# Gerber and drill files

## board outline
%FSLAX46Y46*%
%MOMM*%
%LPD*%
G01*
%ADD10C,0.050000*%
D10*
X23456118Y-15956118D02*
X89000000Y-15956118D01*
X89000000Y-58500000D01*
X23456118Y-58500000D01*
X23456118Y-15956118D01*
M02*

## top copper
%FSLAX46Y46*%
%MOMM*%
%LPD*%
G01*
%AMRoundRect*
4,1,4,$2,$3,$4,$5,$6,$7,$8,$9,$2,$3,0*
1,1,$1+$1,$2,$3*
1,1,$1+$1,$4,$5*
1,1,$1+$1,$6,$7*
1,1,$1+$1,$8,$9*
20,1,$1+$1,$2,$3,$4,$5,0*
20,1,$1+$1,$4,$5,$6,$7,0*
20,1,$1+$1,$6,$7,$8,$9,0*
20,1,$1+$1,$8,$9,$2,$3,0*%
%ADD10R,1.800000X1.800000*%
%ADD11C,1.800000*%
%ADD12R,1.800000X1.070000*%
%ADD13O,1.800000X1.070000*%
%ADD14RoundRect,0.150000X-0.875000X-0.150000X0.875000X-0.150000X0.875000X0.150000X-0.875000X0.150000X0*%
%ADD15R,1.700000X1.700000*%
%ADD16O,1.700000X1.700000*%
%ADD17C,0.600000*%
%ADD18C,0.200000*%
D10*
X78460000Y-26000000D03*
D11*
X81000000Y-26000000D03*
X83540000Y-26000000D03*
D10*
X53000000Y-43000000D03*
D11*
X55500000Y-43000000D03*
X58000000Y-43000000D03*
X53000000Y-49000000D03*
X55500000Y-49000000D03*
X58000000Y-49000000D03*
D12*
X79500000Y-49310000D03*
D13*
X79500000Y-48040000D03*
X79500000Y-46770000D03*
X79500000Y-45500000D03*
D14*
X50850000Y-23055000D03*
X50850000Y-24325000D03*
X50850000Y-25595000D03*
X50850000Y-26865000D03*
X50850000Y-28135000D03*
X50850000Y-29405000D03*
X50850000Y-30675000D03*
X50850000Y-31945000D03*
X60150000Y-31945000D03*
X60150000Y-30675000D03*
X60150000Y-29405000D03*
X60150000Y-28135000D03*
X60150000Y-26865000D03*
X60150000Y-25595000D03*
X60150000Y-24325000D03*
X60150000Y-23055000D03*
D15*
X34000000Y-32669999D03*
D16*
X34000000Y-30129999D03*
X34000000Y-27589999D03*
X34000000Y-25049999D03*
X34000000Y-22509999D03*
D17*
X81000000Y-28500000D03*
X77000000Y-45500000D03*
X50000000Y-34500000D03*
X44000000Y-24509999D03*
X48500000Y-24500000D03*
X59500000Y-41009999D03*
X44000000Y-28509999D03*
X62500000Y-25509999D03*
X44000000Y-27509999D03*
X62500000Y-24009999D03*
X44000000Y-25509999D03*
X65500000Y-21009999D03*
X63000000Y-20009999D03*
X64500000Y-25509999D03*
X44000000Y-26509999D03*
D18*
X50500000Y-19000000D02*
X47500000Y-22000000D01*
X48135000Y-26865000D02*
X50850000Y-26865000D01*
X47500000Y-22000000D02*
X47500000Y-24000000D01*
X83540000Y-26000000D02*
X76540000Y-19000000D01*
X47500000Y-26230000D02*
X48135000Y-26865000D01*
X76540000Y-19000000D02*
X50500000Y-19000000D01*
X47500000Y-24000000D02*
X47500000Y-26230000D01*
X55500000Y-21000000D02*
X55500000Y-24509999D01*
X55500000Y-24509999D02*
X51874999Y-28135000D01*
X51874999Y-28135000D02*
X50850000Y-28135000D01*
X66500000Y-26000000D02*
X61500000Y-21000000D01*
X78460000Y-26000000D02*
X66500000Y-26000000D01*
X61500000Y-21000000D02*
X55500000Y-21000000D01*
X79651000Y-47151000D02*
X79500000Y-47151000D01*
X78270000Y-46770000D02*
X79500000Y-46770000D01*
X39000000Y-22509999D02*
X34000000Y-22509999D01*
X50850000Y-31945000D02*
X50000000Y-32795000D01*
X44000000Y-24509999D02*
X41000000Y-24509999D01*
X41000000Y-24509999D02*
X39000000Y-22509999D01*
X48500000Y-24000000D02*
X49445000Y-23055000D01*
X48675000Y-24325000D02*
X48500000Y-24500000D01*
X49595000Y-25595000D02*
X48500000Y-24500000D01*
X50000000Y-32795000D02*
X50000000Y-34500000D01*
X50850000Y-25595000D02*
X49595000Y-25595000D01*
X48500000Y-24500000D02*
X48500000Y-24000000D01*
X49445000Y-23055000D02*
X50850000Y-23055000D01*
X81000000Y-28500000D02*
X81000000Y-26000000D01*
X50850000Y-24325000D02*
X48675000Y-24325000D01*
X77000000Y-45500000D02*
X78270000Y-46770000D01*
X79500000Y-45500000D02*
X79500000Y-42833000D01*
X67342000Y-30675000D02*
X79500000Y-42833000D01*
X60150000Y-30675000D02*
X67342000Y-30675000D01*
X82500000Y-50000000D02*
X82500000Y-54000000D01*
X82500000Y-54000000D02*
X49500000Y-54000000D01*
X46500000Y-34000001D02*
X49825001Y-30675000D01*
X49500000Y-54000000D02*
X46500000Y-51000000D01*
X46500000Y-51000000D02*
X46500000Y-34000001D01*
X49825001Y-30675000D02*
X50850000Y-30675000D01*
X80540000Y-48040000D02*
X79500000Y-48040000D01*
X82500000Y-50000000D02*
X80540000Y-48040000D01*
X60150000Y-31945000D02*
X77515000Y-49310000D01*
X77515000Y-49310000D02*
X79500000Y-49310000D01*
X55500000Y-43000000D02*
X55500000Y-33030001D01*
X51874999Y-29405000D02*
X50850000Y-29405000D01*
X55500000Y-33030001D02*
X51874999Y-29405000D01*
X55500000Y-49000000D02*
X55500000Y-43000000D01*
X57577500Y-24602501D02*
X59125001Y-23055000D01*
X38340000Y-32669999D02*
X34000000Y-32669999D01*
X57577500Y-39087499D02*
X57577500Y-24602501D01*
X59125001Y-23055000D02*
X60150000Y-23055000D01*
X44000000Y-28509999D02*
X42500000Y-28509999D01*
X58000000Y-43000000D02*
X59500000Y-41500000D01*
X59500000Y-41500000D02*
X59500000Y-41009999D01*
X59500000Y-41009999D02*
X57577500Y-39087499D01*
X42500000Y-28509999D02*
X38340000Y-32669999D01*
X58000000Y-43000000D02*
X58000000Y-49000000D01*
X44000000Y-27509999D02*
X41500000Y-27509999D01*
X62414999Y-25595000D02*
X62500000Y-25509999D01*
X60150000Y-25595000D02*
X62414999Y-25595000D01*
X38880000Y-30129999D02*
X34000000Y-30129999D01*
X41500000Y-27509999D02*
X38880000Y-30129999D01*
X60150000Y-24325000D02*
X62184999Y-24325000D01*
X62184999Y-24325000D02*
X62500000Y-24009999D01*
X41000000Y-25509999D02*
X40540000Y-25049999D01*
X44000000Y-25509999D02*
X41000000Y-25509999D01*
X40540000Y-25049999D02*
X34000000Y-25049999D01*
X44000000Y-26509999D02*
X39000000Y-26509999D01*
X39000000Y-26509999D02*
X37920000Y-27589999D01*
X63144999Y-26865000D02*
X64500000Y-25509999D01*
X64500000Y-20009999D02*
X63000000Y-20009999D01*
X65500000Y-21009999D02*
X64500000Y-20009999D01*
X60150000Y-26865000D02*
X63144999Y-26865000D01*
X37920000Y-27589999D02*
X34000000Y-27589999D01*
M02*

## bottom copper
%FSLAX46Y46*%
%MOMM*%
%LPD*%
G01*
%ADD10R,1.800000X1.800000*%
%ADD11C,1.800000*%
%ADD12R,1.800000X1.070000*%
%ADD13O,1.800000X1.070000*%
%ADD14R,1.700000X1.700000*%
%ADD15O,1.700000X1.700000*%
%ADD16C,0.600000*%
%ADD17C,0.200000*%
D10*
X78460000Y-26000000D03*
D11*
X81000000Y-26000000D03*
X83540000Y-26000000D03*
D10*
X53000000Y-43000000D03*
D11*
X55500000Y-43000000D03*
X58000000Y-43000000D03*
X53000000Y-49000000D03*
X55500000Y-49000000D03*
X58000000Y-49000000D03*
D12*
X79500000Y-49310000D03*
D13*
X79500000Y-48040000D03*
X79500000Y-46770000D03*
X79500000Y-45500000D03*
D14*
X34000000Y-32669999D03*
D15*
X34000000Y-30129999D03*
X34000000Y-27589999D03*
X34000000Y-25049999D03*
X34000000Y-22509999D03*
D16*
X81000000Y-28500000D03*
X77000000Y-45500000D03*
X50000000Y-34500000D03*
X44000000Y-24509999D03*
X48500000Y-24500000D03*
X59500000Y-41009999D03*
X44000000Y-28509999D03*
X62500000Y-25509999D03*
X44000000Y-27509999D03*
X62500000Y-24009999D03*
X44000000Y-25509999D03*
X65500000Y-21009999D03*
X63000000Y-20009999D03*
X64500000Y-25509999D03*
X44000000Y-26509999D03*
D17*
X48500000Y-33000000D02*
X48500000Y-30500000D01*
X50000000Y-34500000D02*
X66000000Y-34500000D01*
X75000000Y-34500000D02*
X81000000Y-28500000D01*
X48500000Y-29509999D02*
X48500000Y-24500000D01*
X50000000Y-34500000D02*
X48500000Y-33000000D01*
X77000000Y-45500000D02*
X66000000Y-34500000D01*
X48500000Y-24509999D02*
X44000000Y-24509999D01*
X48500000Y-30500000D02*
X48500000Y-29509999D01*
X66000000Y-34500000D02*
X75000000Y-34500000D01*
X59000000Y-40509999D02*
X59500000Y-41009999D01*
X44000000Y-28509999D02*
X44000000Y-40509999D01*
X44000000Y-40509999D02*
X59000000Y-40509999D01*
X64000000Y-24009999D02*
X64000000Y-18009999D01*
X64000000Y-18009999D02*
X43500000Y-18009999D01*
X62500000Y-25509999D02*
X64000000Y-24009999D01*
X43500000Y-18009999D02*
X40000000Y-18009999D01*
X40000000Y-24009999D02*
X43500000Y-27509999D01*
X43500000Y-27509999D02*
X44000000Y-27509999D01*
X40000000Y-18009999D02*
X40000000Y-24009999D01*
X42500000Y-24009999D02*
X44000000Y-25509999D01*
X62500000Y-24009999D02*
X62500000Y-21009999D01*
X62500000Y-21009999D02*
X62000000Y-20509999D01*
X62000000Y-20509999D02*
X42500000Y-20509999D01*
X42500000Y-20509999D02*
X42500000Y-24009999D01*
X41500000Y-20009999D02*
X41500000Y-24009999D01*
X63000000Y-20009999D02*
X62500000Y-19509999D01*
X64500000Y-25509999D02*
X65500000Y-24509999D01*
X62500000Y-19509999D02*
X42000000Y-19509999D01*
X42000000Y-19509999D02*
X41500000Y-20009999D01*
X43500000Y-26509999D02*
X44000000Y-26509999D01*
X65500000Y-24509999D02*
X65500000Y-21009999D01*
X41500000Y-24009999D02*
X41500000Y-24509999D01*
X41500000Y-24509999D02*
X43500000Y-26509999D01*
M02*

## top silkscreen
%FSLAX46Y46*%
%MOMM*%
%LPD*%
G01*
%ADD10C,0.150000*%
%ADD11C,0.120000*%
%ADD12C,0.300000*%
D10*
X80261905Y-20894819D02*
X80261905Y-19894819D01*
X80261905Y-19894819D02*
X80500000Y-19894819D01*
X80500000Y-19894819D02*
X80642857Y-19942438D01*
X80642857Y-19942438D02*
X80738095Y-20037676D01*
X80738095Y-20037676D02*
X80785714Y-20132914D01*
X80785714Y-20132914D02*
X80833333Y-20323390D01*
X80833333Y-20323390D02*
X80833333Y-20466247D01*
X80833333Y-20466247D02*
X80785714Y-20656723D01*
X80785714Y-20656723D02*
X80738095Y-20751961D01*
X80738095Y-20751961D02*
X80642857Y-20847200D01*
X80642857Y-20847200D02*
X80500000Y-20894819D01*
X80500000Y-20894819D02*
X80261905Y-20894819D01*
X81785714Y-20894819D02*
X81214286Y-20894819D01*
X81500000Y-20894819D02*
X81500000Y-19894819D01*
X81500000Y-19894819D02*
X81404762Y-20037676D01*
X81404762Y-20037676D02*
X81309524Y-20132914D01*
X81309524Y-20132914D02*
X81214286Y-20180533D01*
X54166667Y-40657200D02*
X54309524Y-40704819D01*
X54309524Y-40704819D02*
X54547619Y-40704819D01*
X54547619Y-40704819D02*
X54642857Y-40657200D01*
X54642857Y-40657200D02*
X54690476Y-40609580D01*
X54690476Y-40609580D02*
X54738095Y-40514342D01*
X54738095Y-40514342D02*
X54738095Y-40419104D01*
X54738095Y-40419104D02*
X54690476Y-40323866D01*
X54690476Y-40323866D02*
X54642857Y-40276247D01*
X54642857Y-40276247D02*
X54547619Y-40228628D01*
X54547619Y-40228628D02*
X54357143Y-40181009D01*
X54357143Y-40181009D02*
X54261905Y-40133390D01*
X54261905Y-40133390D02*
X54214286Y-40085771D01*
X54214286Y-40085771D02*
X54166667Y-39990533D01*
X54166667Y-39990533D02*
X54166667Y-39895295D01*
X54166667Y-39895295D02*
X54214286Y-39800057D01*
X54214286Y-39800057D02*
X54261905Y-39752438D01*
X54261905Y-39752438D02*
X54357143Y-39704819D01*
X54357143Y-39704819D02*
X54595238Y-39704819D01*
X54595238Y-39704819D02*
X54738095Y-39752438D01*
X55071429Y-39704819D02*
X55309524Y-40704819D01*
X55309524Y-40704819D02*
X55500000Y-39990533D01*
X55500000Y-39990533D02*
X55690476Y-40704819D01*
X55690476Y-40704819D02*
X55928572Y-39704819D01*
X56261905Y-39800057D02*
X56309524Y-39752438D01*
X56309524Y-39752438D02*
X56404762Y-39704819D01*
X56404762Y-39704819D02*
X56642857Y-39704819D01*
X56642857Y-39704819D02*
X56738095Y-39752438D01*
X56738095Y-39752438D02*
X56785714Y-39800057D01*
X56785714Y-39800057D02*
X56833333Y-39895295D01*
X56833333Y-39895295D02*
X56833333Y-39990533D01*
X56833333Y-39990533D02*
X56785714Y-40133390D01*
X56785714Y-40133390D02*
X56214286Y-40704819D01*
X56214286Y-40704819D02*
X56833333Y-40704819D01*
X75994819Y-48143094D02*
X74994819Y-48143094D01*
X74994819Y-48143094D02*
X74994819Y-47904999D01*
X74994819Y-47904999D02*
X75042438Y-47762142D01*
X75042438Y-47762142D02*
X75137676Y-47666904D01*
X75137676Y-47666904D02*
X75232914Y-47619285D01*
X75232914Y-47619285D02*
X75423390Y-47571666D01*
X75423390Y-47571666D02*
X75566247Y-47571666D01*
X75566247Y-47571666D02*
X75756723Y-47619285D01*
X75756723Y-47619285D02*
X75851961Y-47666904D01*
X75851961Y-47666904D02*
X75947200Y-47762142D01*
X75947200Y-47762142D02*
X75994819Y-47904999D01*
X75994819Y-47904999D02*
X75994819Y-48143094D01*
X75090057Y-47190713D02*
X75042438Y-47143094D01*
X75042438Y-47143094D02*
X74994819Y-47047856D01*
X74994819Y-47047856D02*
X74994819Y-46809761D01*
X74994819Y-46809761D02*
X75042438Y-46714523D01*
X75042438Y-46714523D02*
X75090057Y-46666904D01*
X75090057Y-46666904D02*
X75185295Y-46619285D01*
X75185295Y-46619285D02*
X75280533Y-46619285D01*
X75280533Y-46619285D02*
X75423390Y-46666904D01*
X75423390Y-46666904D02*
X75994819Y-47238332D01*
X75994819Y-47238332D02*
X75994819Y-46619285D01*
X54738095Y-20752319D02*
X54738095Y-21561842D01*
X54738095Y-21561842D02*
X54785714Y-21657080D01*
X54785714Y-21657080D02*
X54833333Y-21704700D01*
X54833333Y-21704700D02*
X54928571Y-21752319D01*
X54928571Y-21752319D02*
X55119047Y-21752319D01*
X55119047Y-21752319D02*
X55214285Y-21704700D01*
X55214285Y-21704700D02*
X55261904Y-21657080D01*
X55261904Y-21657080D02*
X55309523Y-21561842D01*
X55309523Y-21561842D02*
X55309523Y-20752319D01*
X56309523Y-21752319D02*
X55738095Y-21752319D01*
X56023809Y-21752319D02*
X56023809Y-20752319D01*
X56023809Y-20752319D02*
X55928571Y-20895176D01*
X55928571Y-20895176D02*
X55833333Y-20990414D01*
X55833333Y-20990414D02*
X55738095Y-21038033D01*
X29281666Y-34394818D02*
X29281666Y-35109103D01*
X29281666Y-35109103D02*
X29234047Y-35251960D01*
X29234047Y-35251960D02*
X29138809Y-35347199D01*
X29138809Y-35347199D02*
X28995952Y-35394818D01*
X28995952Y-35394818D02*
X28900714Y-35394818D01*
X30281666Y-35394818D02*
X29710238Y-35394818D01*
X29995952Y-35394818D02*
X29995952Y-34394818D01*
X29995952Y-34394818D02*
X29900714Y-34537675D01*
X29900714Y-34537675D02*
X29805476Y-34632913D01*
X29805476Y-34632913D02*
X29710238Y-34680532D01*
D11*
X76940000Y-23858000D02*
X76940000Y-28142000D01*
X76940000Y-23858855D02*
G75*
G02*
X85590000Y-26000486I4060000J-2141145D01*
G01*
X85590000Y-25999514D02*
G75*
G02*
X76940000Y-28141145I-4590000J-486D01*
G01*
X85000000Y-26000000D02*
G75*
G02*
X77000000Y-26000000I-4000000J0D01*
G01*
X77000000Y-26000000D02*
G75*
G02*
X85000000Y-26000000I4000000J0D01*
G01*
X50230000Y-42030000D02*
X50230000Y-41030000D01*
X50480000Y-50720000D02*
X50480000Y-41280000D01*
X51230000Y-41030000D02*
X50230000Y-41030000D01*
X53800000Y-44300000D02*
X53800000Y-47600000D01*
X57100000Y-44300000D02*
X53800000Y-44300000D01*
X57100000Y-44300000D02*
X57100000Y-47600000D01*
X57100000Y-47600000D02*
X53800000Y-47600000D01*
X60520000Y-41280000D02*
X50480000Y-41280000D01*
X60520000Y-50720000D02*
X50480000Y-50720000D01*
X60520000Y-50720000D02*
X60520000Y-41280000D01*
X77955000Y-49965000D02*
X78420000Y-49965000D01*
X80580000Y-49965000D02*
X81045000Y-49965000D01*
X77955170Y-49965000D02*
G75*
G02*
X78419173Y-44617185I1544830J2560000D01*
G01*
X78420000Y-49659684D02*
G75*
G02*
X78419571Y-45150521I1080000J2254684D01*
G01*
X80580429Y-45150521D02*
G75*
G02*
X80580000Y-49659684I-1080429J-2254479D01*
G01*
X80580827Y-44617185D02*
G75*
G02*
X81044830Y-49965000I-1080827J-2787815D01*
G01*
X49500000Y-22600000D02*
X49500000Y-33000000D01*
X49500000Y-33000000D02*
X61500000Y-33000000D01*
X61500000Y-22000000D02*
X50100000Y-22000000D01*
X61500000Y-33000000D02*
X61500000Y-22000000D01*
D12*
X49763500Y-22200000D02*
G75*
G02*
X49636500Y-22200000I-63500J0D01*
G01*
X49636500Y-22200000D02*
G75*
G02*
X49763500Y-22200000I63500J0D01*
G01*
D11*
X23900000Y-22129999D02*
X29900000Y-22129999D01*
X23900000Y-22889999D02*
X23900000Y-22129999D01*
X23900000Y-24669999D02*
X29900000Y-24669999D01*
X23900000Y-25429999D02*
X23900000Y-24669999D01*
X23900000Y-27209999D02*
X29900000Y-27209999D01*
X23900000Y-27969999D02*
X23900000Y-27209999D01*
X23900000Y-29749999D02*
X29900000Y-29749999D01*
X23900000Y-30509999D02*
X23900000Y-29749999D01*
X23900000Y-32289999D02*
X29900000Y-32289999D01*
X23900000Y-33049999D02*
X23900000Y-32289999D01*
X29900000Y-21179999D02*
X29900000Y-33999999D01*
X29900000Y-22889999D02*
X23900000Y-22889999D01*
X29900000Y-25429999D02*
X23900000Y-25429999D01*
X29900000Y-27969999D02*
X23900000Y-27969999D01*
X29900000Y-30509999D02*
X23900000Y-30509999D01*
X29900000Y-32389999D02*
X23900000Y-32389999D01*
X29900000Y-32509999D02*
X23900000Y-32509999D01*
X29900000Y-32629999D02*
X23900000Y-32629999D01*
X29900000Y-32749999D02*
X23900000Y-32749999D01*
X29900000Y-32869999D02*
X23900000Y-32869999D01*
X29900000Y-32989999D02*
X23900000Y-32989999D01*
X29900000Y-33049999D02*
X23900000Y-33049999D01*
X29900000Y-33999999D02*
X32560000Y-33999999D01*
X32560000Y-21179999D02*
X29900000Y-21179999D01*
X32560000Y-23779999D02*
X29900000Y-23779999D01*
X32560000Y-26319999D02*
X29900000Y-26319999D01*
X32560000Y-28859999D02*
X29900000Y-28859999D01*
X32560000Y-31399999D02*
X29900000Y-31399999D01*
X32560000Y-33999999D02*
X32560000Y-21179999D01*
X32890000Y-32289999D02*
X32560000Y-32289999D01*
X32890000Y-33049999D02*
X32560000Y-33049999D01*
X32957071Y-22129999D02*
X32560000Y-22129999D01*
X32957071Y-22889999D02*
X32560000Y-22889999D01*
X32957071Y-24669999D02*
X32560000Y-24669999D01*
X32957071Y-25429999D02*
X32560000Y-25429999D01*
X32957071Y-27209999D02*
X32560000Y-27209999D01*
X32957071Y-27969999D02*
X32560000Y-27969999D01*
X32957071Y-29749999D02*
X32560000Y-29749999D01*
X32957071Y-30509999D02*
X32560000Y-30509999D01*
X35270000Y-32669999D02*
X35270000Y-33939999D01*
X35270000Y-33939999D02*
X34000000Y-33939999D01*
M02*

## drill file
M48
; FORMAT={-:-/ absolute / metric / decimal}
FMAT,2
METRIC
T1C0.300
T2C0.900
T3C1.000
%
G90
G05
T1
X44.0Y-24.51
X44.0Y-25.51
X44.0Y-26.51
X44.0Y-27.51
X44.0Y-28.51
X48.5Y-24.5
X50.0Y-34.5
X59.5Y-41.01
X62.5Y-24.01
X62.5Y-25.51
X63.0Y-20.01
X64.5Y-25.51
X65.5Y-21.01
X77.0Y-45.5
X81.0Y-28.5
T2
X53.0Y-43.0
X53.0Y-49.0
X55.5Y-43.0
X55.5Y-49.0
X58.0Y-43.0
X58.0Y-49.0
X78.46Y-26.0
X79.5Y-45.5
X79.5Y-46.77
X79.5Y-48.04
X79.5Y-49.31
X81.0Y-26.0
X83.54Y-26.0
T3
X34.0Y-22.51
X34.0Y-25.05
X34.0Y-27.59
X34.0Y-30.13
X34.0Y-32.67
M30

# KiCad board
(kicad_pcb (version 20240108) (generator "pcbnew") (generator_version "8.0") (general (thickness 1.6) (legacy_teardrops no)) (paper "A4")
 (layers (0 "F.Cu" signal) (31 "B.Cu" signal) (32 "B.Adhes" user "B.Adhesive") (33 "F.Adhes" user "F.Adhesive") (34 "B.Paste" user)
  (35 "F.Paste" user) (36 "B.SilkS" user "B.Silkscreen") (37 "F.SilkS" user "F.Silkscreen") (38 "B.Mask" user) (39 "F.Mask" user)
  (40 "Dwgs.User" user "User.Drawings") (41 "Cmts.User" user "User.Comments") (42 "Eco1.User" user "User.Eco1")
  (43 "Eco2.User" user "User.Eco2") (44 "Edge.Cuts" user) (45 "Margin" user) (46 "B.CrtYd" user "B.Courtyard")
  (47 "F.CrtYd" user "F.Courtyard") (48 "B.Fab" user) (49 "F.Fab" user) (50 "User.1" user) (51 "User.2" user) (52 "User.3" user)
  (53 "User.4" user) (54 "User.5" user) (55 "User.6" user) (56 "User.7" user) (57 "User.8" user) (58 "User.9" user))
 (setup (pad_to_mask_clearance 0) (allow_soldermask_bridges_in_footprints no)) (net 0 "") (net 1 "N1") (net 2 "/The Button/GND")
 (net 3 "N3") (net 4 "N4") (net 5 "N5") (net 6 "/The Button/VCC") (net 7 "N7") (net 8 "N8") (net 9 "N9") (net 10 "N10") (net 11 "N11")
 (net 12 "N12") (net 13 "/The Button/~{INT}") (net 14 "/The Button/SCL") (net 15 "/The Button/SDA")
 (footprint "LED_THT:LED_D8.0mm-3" (layer "F.Cu") (at 78.46 26)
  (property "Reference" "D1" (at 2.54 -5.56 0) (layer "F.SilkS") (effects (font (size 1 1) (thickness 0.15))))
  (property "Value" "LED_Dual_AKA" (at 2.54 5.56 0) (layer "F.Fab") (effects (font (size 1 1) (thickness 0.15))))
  (fp_line (start -1.52 -2.142) (end -1.52 2.142) (stroke (width 0.12) (type solid)) (layer "F.SilkS"))
  (fp_arc (start -1.52 -2.141145) (mid 3.643119 -4.455472) (end 7.13 0.000486) (stroke (width 0.12) (type solid)) (layer "F.SilkS"))
  (fp_arc (start 7.13 -0.000486) (mid 3.643119 4.455472) (end -1.52 2.141145) (stroke (width 0.12) (type solid)) (layer "F.SilkS"))
  (fp_circle (center 2.54 0) (end 6.54 0) (stroke (width 0.12) (type solid)) (fill none) (layer "F.SilkS"))
  (pad "1" thru_hole rect (at 0 0) (size 1.8 1.8) (drill 0.9) (layers "*.Cu" "*.Mask") (remove_unused_layers no) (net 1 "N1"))
  (pad "2" thru_hole circle (at 2.54 0) (size 1.8 1.8) (drill 0.9) (layers "*.Cu" "*.Mask") (remove_unused_layers no)
   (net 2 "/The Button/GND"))
  (pad "3" thru_hole circle (at 5.08 0) (size 1.8 1.8) (drill 0.9) (layers "*.Cu" "*.Mask") (remove_unused_layers no) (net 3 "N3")))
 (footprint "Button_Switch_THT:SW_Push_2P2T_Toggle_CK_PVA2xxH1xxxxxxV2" (layer "F.Cu") (at 53 43)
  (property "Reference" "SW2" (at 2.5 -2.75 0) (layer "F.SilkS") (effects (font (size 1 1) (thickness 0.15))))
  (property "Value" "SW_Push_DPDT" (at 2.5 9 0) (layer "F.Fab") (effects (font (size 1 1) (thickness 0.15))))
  (fp_line (start -2.77 -0.97) (end -2.77 -1.97) (stroke (width 0.12) (type solid)) (layer "F.SilkS"))
  (fp_line (start -2.52 7.72) (end -2.52 -1.72) (stroke (width 0.12) (type solid)) (layer "F.SilkS"))
  (fp_line (start -1.77 -1.97) (end -2.77 -1.97) (stroke (width 0.12) (type solid)) (layer "F.SilkS"))
  (fp_line (start 0.8 1.3) (end 0.8 4.6) (stroke (width 0.12) (type solid)) (layer "F.SilkS"))
  (fp_line (start 4.1 1.3) (end 0.8 1.3) (stroke (width 0.12) (type solid)) (layer "F.SilkS"))
  (fp_line (start 4.1 1.3) (end 4.1 4.6) (stroke (width 0.12) (type solid)) (layer "F.SilkS"))
  (fp_line (start 4.1 4.6) (end 0.8 4.6) (stroke (width 0.12) (type solid)) (layer "F.SilkS"))
  (fp_line (start 7.52 -1.72) (end -2.52 -1.72) (stroke (width 0.12) (type solid)) (layer "F.SilkS"))
  (fp_line (start 7.52 7.72) (end -2.52 7.72) (stroke (width 0.12) (type solid)) (layer "F.SilkS"))
  (fp_line (start 7.52 7.72) (end 7.52 -1.72) (stroke (width 0.12) (type solid)) (layer "F.SilkS"))
  (pad "1" thru_hole rect (at 0 0) (size 1.8 1.8) (drill 0.9) (layers "*.Cu" "*.Mask") (remove_unused_layers no) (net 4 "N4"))
  (pad "2" thru_hole circle (at 2.5 0) (size 1.8 1.8) (drill 0.9) (layers "*.Cu" "*.Mask") (remove_unused_layers no) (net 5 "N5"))
  (pad "3" thru_hole circle (at 5 0) (size 1.8 1.8) (drill 0.9) (layers "*.Cu" "*.Mask") (remove_unused_layers no) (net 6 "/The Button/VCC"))
  (pad "4" thru_hole circle (at 0 6) (size 1.8 1.8) (drill 0.9) (layers "*.Cu" "*.Mask") (remove_unused_layers no) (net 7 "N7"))
  (pad "5" thru_hole circle (at 2.5 6) (size 1.8 1.8) (drill 0.9) (layers "*.Cu" "*.Mask") (remove_unused_layers no) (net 5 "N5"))
  (pad "6" thru_hole circle (at 5 6) (size 1.8 1.8) (drill 0.9) (layers "*.Cu" "*.Mask") (remove_unused_layers no) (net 6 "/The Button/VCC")))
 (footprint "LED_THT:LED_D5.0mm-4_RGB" (layer "F.Cu") (at 79.5 49.31 90)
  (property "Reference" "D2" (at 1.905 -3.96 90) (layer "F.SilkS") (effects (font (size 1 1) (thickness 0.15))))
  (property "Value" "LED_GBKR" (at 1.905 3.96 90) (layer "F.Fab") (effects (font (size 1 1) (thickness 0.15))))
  (fp_line (start -0.655 -1.545) (end -0.655 -1.08) (stroke (width 0.12) (type solid)) (layer "F.SilkS"))
  (fp_line (start -0.655 1.08) (end -0.655 1.545) (stroke (width 0.12) (type solid)) (layer "F.SilkS"))
  (fp_arc (start -0.655 -1.54483) (mid 2.163456 -2.978809) (end 4.692815 -1.080827) (stroke (width 0.12) (type solid)) (layer "F.SilkS"))
  (fp_arc (start -0.349684 -1.08) (mid 1.904762 -2.5) (end 4.159479 -1.080429) (stroke (width 0.12) (type solid)) (layer "F.SilkS"))
  (fp_arc (start 4.159479 1.080429) (mid 1.904762 2.5) (end -0.349684 1.08) (stroke (width 0.12) (type solid)) (layer "F.SilkS"))
  (fp_arc (start 4.692815 1.080827) (mid 2.163456 2.978808) (end -0.655 1.54483) (stroke (width 0.12) (type solid)) (layer "F.SilkS"))
  (pad "1" thru_hole rect (at 0 0 90) (size 1.07 1.8) (drill 0.9) (layers "*.Cu" "*.Mask") (remove_unused_layers no) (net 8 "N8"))
  (pad "2" thru_hole oval (at 1.27 0 90) (size 1.07 1.8) (drill 0.9) (layers "*.Cu" "*.Mask") (remove_unused_layers no) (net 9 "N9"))
  (pad "3" thru_hole oval (at 2.54 0 90) (size 1.07 1.8) (drill 0.9) (layers "*.Cu" "*.Mask") (remove_unused_layers no)
   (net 2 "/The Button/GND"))
  (pad "4" thru_hole oval (at 3.81 0 90) (size 1.07 1.8) (drill 0.9) (layers "*.Cu" "*.Mask") (remove_unused_layers no) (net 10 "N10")))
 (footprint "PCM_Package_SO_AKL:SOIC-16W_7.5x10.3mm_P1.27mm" (layer "F.Cu") (at 55.5 27.5)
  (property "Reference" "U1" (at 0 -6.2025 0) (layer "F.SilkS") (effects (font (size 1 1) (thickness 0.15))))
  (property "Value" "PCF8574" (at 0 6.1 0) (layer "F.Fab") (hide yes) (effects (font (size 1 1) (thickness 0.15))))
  (fp_line (start -6 -4.9) (end -6 5.5) (stroke (width 0.12) (type solid)) (layer "F.SilkS"))
  (fp_line (start -6 5.5) (end 6 5.5) (stroke (width 0.12) (type solid)) (layer "F.SilkS"))
  (fp_line (start 6 -5.5) (end -5.4 -5.5) (stroke (width 0.12) (type solid)) (layer "F.SilkS"))
  (fp_line (start 6 5.5) (end 6 -5.5) (stroke (width 0.12) (type solid)) (layer "F.SilkS"))
  (fp_circle (center -5.8 -5.3) (end -5.7365 -5.3) (stroke (width 0.3) (type solid)) (fill none) (layer "F.SilkS"))
  (pad "1" smd roundrect (at -4.65 -4.445) (size 2.05 0.6) (layers "F.Cu" "F.Paste" "F.Mask") (roundrect_rratio 0.25)
   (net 2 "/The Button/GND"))
  (pad "2" smd roundrect (at -4.65 -3.175) (size 2.05 0.6) (layers "F.Cu" "F.Paste" "F.Mask") (roundrect_rratio 0.25)
   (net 2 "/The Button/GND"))
  (pad "3" smd roundrect (at -4.65 -1.905) (size 2.05 0.6) (layers "F.Cu" "F.Paste" "F.Mask") (roundrect_rratio 0.25)
   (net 2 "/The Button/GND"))
  (pad "4" smd roundrect (at -4.65 -0.635) (size 2.05 0.6) (layers "F.Cu" "F.Paste" "F.Mask") (roundrect_rratio 0.25) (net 3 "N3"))
  (pad "5" smd roundrect (at -4.65 0.635) (size 2.05 0.6) (layers "F.Cu" "F.Paste" "F.Mask") (roundrect_rratio 0.25) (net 1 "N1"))
  (pad "6" smd roundrect (at -4.65 1.905) (size 2.05 0.6) (layers "F.Cu" "F.Paste" "F.Mask") (roundrect_rratio 0.25) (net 5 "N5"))
  (pad "7" smd roundrect (at -4.65 3.175) (size 2.05 0.6) (layers "F.Cu" "F.Paste" "F.Mask") (roundrect_rratio 0.25) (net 9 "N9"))
  (pad "8" smd roundrect (at -4.65 4.445) (size 2.05 0.6) (layers "F.Cu" "F.Paste" "F.Mask") (roundrect_rratio 0.25)
   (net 2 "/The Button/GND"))
  (pad "9" smd roundrect (at 4.65 4.445) (size 2.05 0.6) (layers "F.Cu" "F.Paste" "F.Mask") (roundrect_rratio 0.25) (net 8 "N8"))
  (pad "10" smd roundrect (at 4.65 3.175) (size 2.05 0.6) (layers "F.Cu" "F.Paste" "F.Mask") (roundrect_rratio 0.25) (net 10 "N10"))
  (pad "11" smd roundrect (at 4.65 1.905) (size 2.05 0.6) (layers "F.Cu" "F.Paste" "F.Mask") (roundrect_rratio 0.25) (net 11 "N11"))
  (pad "12" smd roundrect (at 4.65 0.635) (size 2.05 0.6) (layers "F.Cu" "F.Paste" "F.Mask") (roundrect_rratio 0.25) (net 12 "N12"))
  (pad "13" smd roundrect (at 4.65 -0.635) (size 2.05 0.6) (layers "F.Cu" "F.Paste" "F.Mask") (roundrect_rratio 0.25)
   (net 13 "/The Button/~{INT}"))
  (pad "14" smd roundrect (at 4.65 -1.905) (size 2.05 0.6) (layers "F.Cu" "F.Paste" "F.Mask") (roundrect_rratio 0.25)
   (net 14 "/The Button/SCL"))
  (pad "15" smd roundrect (at 4.65 -3.175) (size 2.05 0.6) (layers "F.Cu" "F.Paste" "F.Mask") (roundrect_rratio 0.25)
   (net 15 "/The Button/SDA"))
  (pad "16" smd roundrect (at 4.65 -4.445) (size 2.05 0.6) (layers "F.Cu" "F.Paste" "F.Mask") (roundrect_rratio 0.25)
   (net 6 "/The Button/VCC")))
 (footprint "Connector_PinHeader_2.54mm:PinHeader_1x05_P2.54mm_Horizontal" (layer "F.Cu") (at 34 32.669999 180)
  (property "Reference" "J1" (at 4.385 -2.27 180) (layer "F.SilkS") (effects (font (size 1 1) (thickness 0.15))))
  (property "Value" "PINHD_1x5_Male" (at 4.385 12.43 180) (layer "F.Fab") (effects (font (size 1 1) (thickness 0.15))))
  (fp_line (start 10.1 10.54) (end 4.1 10.54) (stroke (width 0.12) (type solid)) (layer "F.SilkS"))
  (fp_line (start 10.1 9.78) (end 10.1 10.54) (stroke (width 0.12) (type solid)) (layer "F.SilkS"))
  (fp_line (start 10.1 8) (end 4.1 8) (stroke (width 0.12) (type solid)) (layer "F.SilkS"))
  (fp_line (start 10.1 7.24) (end 10.1 8) (stroke (width 0.12) (type solid)) (layer "F.SilkS"))
  (fp_line (start 10.1 5.46) (end 4.1 5.46) (stroke (width 0.12) (type solid)) (layer "F.SilkS"))
  (fp_line (start 10.1 4.7) (end 10.1 5.46) (stroke (width 0.12) (type solid)) (layer "F.SilkS"))
  (fp_line (start 10.1 2.92) (end 4.1 2.92) (stroke (width 0.12) (type solid)) (layer "F.SilkS"))
  (fp_line (start 10.1 2.16) (end 10.1 2.92) (stroke (width 0.12) (type solid)) (layer "F.SilkS"))
  (fp_line (start 10.1 0.38) (end 4.1 0.38) (stroke (width 0.12) (type solid)) (layer "F.SilkS"))
  (fp_line (start 10.1 -0.38) (end 10.1 0.38) (stroke (width 0.12) (type solid)) (layer "F.SilkS"))
  (fp_line (start 4.1 11.49) (end 4.1 -1.33) (stroke (width 0.12) (type solid)) (layer "F.SilkS"))
  (fp_line (start 4.1 9.78) (end 10.1 9.78) (stroke (width 0.12) (type solid)) (layer "F.SilkS"))
  (fp_line (start 4.1 7.24) (end 10.1 7.24) (stroke (width 0.12) (type solid)) (layer "F.SilkS"))
  (fp_line (start 4.1 4.7) (end 10.1 4.7) (stroke (width 0.12) (type solid)) (layer "F.SilkS"))
  (fp_line (start 4.1 2.16) (end 10.1 2.16) (stroke (width 0.12) (type solid)) (layer "F.SilkS"))
  (fp_line (start 4.1 0.28) (end 10.1 0.28) (stroke (width 0.12) (type solid)) (layer "F.SilkS"))
  (fp_line (start 4.1 0.16) (end 10.1 0.16) (stroke (width 0.12) (type solid)) (layer "F.SilkS"))
  (fp_line (start 4.1 0.04) (end 10.1 0.04) (stroke (width 0.12) (type solid)) (layer "F.SilkS"))
  (fp_line (start 4.1 -0.08) (end 10.1 -0.08) (stroke (width 0.12) (type solid)) (layer "F.SilkS"))
  (fp_line (start 4.1 -0.2) (end 10.1 -0.2) (stroke (width 0.12) (type solid)) (layer "F.SilkS"))
  (fp_line (start 4.1 -0.32) (end 10.1 -0.32) (stroke (width 0.12) (type solid)) (layer "F.SilkS"))
  (fp_line (start 4.1 -0.38) (end 10.1 -0.38) (stroke (width 0.12) (type solid)) (layer "F.SilkS"))
  (fp_line (start 4.1 -1.33) (end 1.44 -1.33) (stroke (width 0.12) (type solid)) (layer "F.SilkS"))
  (fp_line (start 1.44 11.49) (end 4.1 11.49) (stroke (width 0.12) (type solid)) (layer "F.SilkS"))
  (fp_line (start 1.44 8.89) (end 4.1 8.89) (stroke (width 0.12) (type solid)) (layer "F.SilkS"))
  (fp_line (start 1.44 6.35) (end 4.1 6.35) (stroke (width 0.12) (type solid)) (layer "F.SilkS"))
  (fp_line (start 1.44 3.81) (end 4.1 3.81) (stroke (width 0.12) (type solid)) (layer "F.SilkS"))
  (fp_line (start 1.44 1.27) (end 4.1 1.27) (stroke (width 0.12) (type solid)) (layer "F.SilkS"))
  (fp_line (start 1.44 -1.33) (end 1.44 11.49) (stroke (width 0.12) (type solid)) (layer "F.SilkS"))
  (fp_line (start 1.11 0.38) (end 1.44 0.38) (stroke (width 0.12) (type solid)) (layer "F.SilkS"))
  (fp_line (start 1.11 -0.38) (end 1.44 -0.38) (stroke (width 0.12) (type solid)) (layer "F.SilkS"))
  (fp_line (start 1.042929 10.54) (end 1.44 10.54) (stroke (width 0.12) (type solid)) (layer "F.SilkS"))
  (fp_line (start 1.042929 9.78) (end 1.44 9.78) (stroke (width 0.12) (type solid)) (layer "F.SilkS"))
  (fp_line (start 1.042929 8) (end 1.44 8) (stroke (width 0.12) (type solid)) (layer "F.SilkS"))
  (fp_line (start 1.042929 7.24) (end 1.44 7.24) (stroke (width 0.12) (type solid)) (layer "F.SilkS"))
  (fp_line (start 1.042929 5.46) (end 1.44 5.46) (stroke (width 0.12) (type solid)) (layer "F.SilkS"))
  (fp_line (start 1.042929 4.7) (end 1.44 4.7) (stroke (width 0.12) (type solid)) (layer "F.SilkS"))
  (fp_line (start 1.042929 2.92) (end 1.44 2.92) (stroke (width 0.12) (type solid)) (layer "F.SilkS"))
  (fp_line (start 1.042929 2.16) (end 1.44 2.16) (stroke (width 0.12) (type solid)) (layer "F.SilkS"))
  (fp_line (start -1.27 0) (end -1.27 -1.27) (stroke (width 0.12) (type solid)) (layer "F.SilkS"))
  (fp_line (start -1.27 -1.27) (end 0 -1.27) (stroke (width 0.12) (type solid)) (layer "F.SilkS"))
  (pad "1" thru_hole rect (at 0 0 180) (size 1.7 1.7) (drill 1) (layers "*.Cu" "*.Mask") (remove_unused_layers no) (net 6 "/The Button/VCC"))
  (pad "2" thru_hole oval (at 0 2.54 180) (size 1.7 1.7) (drill 1) (layers "*.Cu" "*.Mask") (remove_unused_layers no)
   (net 14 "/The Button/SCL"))
  (pad "3" thru_hole oval (at 0 5.08 180) (size 1.7 1.7) (drill 1) (layers "*.Cu" "*.Mask") (remove_unused_layers no)
   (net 13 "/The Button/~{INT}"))
  (pad "4" thru_hole oval (at 0 7.62 180) (size 1.7 1.7) (drill 1) (layers "*.Cu" "*.Mask") (remove_unused_layers no)
   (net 15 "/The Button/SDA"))
  (pad "5" thru_hole oval (at 0 10.16 180) (size 1.7 1.7) (drill 1) (layers "*.Cu" "*.Mask") (remove_unused_layers no)
   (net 2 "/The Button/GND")))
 (gr_rect (start 23.456118 15.956118) (end 89 58.5) (stroke (width 0.05) (type default)) (fill none) (layer "Edge.Cuts"))
 (segment (start 50.5 19) (end 47.5 22) (width 0.2) (layer "F.Cu") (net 3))
 (segment (start 48.135 26.865) (end 50.85 26.865) (width 0.2) (layer "F.Cu") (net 3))
 (segment (start 47.5 22) (end 47.5 24) (width 0.2) (layer "F.Cu") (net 3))
 (segment (start 83.54 26) (end 76.54 19) (width 0.2) (layer "F.Cu") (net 3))
 (segment (start 47.5 26.23) (end 48.135 26.865) (width 0.2) (layer "F.Cu") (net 3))
 (segment (start 76.54 19) (end 50.5 19) (width 0.2) (layer "F.Cu") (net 3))
 (segment (start 47.5 24) (end 47.5 26.23) (width 0.2) (layer "F.Cu") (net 3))
 (segment (start 55.5 21) (end 55.5 24.509999) (width 0.2) (layer "F.Cu") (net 1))
 (segment (start 55.5 24.509999) (end 51.874999 28.135) (width 0.2) (layer "F.Cu") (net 1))
 (segment (start 51.874999 28.135) (end 50.85 28.135) (width 0.2) (layer "F.Cu") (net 1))
 (segment (start 66.5 26) (end 61.5 21) (width 0.2) (layer "F.Cu") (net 1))
 (segment (start 78.46 26) (end 66.5 26) (width 0.2) (layer "F.Cu") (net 1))
 (segment (start 61.5 21) (end 55.5 21) (width 0.2) (layer "F.Cu") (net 1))
 (segment (start 79.651 47.151) (end 79.5 47.151) (width 0.2) (layer "F.Cu") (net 2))
 (segment (start 78.27 46.77) (end 79.5 46.77) (width 0.2) (layer "F.Cu") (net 2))
 (segment (start 39 22.509999) (end 34 22.509999) (width 0.2) (layer "F.Cu") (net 2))
 (segment (start 50.85 31.945) (end 50 32.795) (width 0.2) (layer "F.Cu") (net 2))
 (segment (start 44 24.509999) (end 41 24.509999) (width 0.2) (layer "F.Cu") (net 2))
 (segment (start 41 24.509999) (end 39 22.509999) (width 0.2) (layer "F.Cu") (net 2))
 (segment (start 48.5 24) (end 49.445 23.055) (width 0.2) (layer "F.Cu") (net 2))
 (segment (start 48.675 24.325) (end 48.5 24.5) (width 0.2) (layer "F.Cu") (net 2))
 (segment (start 49.595 25.595) (end 48.5 24.5) (width 0.2) (layer "F.Cu") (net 2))
 (segment (start 50 32.795) (end 50 34.5) (width 0.2) (layer "F.Cu") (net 2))
 (segment (start 50.85 25.595) (end 49.595 25.595) (width 0.2) (layer "F.Cu") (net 2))
 (segment (start 48.5 24.5) (end 48.5 24) (width 0.2) (layer "F.Cu") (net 2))
 (segment (start 49.445 23.055) (end 50.85 23.055) (width 0.2) (layer "F.Cu") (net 2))
 (segment (start 81 28.5) (end 81 26) (width 0.2) (layer "F.Cu") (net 2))
 (segment (start 50.85 24.325) (end 48.675 24.325) (width 0.2) (layer "F.Cu") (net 2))
 (segment (start 77 45.5) (end 78.27 46.77) (width 0.2) (layer "F.Cu") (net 2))
 (via (at 81 28.5) (size 0.6) (drill 0.3) (layers "F.Cu" "B.Cu") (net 2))
 (via (at 77 45.5) (size 0.6) (drill 0.3) (layers "F.Cu" "B.Cu") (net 2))
 (via (at 50 34.5) (size 0.6) (drill 0.3) (layers "F.Cu" "B.Cu") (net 2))
 (via (at 44 24.509999) (size 0.6) (drill 0.3) (layers "F.Cu" "B.Cu") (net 2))
 (via (at 48.5 24.5) (size 0.6) (drill 0.3) (layers "F.Cu" "B.Cu") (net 2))
 (segment (start 48.5 33) (end 48.5 30.5) (width 0.2) (layer "B.Cu") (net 2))
 (segment (start 50 34.5) (end 66 34.5) (width 0.2) (layer "B.Cu") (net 2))
 (segment (start 75 34.5) (end 81 28.5) (width 0.2) (layer "B.Cu") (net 2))
 (segment (start 48.5 29.509999) (end 48.5 24.5) (width 0.2) (layer "B.Cu") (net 2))
 (segment (start 50 34.5) (end 48.5 33) (width 0.2) (layer "B.Cu") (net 2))
 (segment (start 77 45.5) (end 66 34.5) (width 0.2) (layer "B.Cu") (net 2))
 (segment (start 48.5 24.509999) (end 44 24.509999) (width 0.2) (layer "B.Cu") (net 2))
 (segment (start 48.5 30.5) (end 48.5 29.509999) (width 0.2) (layer "B.Cu") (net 2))
 (segment (start 66 34.5) (end 75 34.5) (width 0.2) (layer "B.Cu") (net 2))
 (segment (start 79.5 45.5) (end 79.5 42.833) (width 0.2) (layer "F.Cu") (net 10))
 (segment (start 67.342 30.675) (end 79.5 42.833) (width 0.2) (layer "F.Cu") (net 10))
 (segment (start 60.15 30.675) (end 67.342 30.675) (width 0.2) (layer "F.Cu") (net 10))
 (segment (start 82.5 50) (end 82.5 54) (width 0.2) (layer "F.Cu") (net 9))
 (segment (start 82.5 54) (end 49.5 54) (width 0.2) (layer "F.Cu") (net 9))
 (segment (start 46.5 34.000001) (end 49.825001 30.675) (width 0.2) (layer "F.Cu") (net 9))
 (segment (start 49.5 54) (end 46.5 51) (width 0.2) (layer "F.Cu") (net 9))
 (segment (start 46.5 51) (end 46.5 34.000001) (width 0.2) (layer "F.Cu") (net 9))
 (segment (start 49.825001 30.675) (end 50.85 30.675) (width 0.2) (layer "F.Cu") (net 9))
 (segment (start 80.54 48.04) (end 79.5 48.04) (width 0.2) (layer "F.Cu") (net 9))
 (segment (start 82.5 50) (end 80.54 48.04) (width 0.2) (layer "F.Cu") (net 9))
 (segment (start 60.15 31.945) (end 77.515 49.31) (width 0.2) (layer "F.Cu") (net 8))
 (segment (start 77.515 49.31) (end 79.5 49.31) (width 0.2) (layer "F.Cu") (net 8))
 (segment (start 55.5 43) (end 55.5 33.030001) (width 0.2) (layer "F.Cu") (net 5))
 (segment (start 51.874999 29.405) (end 50.85 29.405) (width 0.2) (layer "F.Cu") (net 5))
 (segment (start 55.5 33.030001) (end 51.874999 29.405) (width 0.2) (layer "F.Cu") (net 5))
 (segment (start 55.5 49) (end 55.5 43) (width 0.2) (layer "F.Cu") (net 5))
 (segment (start 57.5775 24.602501) (end 59.125001 23.055) (width 0.2) (layer "F.Cu") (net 6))
 (segment (start 38.34 32.669999) (end 34 32.669999) (width 0.2) (layer "F.Cu") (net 6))
 (segment (start 57.5775 39.087499) (end 57.5775 24.602501) (width 0.2) (layer "F.Cu") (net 6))
 (segment (start 59.125001 23.055) (end 60.15 23.055) (width 0.2) (layer "F.Cu") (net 6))
 (segment (start 44 28.509999) (end 42.5 28.509999) (width 0.2) (layer "F.Cu") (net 6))
 (segment (start 58 43) (end 59.5 41.5) (width 0.2) (layer "F.Cu") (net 6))
 (segment (start 59.5 41.5) (end 59.5 41.009999) (width 0.2) (layer "F.Cu") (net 6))
 (segment (start 59.5 41.009999) (end 57.5775 39.087499) (width 0.2) (layer "F.Cu") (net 6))
 (segment (start 42.5 28.509999) (end 38.34 32.669999) (width 0.2) (layer "F.Cu") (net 6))
 (segment (start 58 43) (end 58 49) (width 0.2) (layer "F.Cu") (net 6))
 (via (at 59.5 41.009999) (size 0.6) (drill 0.3) (layers "F.Cu" "B.Cu") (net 6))
 (via (at 44 28.509999) (size 0.6) (drill 0.3) (layers "F.Cu" "B.Cu") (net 6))
 (segment (start 59 40.509999) (end 59.5 41.009999) (width 0.2) (layer "B.Cu") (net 6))
 (segment (start 44 28.509999) (end 44 40.509999) (width 0.2) (layer "B.Cu") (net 6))
 (segment (start 44 40.509999) (end 59 40.509999) (width 0.2) (layer "B.Cu") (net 6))
 (segment (start 44 27.509999) (end 41.5 27.509999) (width 0.2) (layer "F.Cu") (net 14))
 (segment (start 62.414999 25.595) (end 62.5 25.509999) (width 0.2) (layer "F.Cu") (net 14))
 (segment (start 60.15 25.595) (end 62.414999 25.595) (width 0.2) (layer "F.Cu") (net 14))
 (segment (start 38.88 30.129999) (end 34 30.129999) (width 0.2) (layer "F.Cu") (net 14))
 (segment (start 41.5 27.509999) (end 38.88 30.129999) (width 0.2) (layer "F.Cu") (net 14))
 (via (at 62.5 25.509999) (size 0.6) (drill 0.3) (layers "F.Cu" "B.Cu") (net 14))
 (via (at 44 27.509999) (size 0.6) (drill 0.3) (layers "F.Cu" "B.Cu") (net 14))
 (segment (start 64 24.009999) (end 64 18.009999) (width 0.2) (layer "B.Cu") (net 14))
 (segment (start 64 18.009999) (end 43.5 18.009999) (width 0.2) (layer "B.Cu") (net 14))
 (segment (start 62.5 25.509999) (end 64 24.009999) (width 0.2) (layer "B.Cu") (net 14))
 (segment (start 43.5 18.009999) (end 40 18.009999) (width 0.2) (layer "B.Cu") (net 14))
 (segment (start 40 24.009999) (end 43.5 27.509999) (width 0.2) (layer "B.Cu") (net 14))
 (segment (start 43.5 27.509999) (end 44 27.509999) (width 0.2) (layer "B.Cu") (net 14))
 (segment (start 40 18.009999) (end 40 24.009999) (width 0.2) (layer "B.Cu") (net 14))
 (segment (start 60.15 24.325) (end 62.184999 24.325) (width 0.2) (layer "F.Cu") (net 15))
 (segment (start 62.184999 24.325) (end 62.5 24.009999) (width 0.2) (layer "F.Cu") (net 15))
 (segment (start 41 25.509999) (end 40.54 25.049999) (width 0.2) (layer "F.Cu") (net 15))
 (segment (start 44 25.509999) (end 41 25.509999) (width 0.2) (layer "F.Cu") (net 15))
 (segment (start 40.54 25.049999) (end 34 25.049999) (width 0.2) (layer "F.Cu") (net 15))
 (via (at 62.5 24.009999) (size 0.6) (drill 0.3) (layers "F.Cu" "B.Cu") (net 15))
 (via (at 44 25.509999) (size 0.6) (drill 0.3) (layers "F.Cu" "B.Cu") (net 15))
 (segment (start 42.5 24.009999) (end 44 25.509999) (width 0.2) (layer "B.Cu") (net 15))
 (segment (start 62.5 24.009999) (end 62.5 21.009999) (width 0.2) (layer "B.Cu") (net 15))
 (segment (start 62.5 21.009999) (end 62 20.509999) (width 0.2) (layer "B.Cu") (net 15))
 (segment (start 62 20.509999) (end 42.5 20.509999) (width 0.2) (layer "B.Cu") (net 15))
 (segment (start 42.5 20.509999) (end 42.5 24.009999) (width 0.2) (layer "B.Cu") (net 15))
 (segment (start 44 26.509999) (end 39 26.509999) (width 0.2) (layer "F.Cu") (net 13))
 (segment (start 39 26.509999) (end 37.92 27.589999) (width 0.2) (layer "F.Cu") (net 13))
 (segment (start 63.144999 26.865) (end 64.5 25.509999) (width 0.2) (layer "F.Cu") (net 13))
 (segment (start 64.5 20.009999) (end 63 20.009999) (width 0.2) (layer "F.Cu") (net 13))
 (segment (start 65.5 21.009999) (end 64.5 20.009999) (width 0.2) (layer "F.Cu") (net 13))
 (segment (start 60.15 26.865) (end 63.144999 26.865) (width 0.2) (layer "F.Cu") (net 13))
 (segment (start 37.92 27.589999) (end 34 27.589999) (width 0.2) (layer "F.Cu") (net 13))
 (via (at 65.5 21.009999) (size 0.6) (drill 0.3) (layers "F.Cu" "B.Cu") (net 13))
 (via (at 63 20.009999) (size 0.6) (drill 0.3) (layers "F.Cu" "B.Cu") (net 13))
 (via (at 64.5 25.509999) (size 0.6) (drill 0.3) (layers "F.Cu" "B.Cu") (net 13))
 (via (at 44 26.509999) (size 0.6) (drill 0.3) (layers "F.Cu" "B.Cu") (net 13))
 (segment (start 41.5 20.009999) (end 41.5 24.009999) (width 0.2) (layer "B.Cu") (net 13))
 (segment (start 63 20.009999) (end 62.5 19.509999) (width 0.2) (layer "B.Cu") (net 13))
 (segment (start 64.5 25.509999) (end 65.5 24.509999) (width 0.2) (layer "B.Cu") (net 13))
 (segment (start 62.5 19.509999) (end 42 19.509999) (width 0.2) (layer "B.Cu") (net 13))
 (segment (start 42 19.509999) (end 41.5 20.009999) (width 0.2) (layer "B.Cu") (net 13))
 (segment (start 43.5 26.509999) (end 44 26.509999) (width 0.2) (layer "B.Cu") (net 13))
 (segment (start 65.5 24.509999) (end 65.5 21.009999) (width 0.2) (layer "B.Cu") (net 13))
 (segment (start 41.5 24.009999) (end 41.5 24.509999) (width 0.2) (layer "B.Cu") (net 13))
 (segment (start 41.5 24.509999) (end 43.5 26.509999) (width 0.2) (layer "B.Cu") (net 13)))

